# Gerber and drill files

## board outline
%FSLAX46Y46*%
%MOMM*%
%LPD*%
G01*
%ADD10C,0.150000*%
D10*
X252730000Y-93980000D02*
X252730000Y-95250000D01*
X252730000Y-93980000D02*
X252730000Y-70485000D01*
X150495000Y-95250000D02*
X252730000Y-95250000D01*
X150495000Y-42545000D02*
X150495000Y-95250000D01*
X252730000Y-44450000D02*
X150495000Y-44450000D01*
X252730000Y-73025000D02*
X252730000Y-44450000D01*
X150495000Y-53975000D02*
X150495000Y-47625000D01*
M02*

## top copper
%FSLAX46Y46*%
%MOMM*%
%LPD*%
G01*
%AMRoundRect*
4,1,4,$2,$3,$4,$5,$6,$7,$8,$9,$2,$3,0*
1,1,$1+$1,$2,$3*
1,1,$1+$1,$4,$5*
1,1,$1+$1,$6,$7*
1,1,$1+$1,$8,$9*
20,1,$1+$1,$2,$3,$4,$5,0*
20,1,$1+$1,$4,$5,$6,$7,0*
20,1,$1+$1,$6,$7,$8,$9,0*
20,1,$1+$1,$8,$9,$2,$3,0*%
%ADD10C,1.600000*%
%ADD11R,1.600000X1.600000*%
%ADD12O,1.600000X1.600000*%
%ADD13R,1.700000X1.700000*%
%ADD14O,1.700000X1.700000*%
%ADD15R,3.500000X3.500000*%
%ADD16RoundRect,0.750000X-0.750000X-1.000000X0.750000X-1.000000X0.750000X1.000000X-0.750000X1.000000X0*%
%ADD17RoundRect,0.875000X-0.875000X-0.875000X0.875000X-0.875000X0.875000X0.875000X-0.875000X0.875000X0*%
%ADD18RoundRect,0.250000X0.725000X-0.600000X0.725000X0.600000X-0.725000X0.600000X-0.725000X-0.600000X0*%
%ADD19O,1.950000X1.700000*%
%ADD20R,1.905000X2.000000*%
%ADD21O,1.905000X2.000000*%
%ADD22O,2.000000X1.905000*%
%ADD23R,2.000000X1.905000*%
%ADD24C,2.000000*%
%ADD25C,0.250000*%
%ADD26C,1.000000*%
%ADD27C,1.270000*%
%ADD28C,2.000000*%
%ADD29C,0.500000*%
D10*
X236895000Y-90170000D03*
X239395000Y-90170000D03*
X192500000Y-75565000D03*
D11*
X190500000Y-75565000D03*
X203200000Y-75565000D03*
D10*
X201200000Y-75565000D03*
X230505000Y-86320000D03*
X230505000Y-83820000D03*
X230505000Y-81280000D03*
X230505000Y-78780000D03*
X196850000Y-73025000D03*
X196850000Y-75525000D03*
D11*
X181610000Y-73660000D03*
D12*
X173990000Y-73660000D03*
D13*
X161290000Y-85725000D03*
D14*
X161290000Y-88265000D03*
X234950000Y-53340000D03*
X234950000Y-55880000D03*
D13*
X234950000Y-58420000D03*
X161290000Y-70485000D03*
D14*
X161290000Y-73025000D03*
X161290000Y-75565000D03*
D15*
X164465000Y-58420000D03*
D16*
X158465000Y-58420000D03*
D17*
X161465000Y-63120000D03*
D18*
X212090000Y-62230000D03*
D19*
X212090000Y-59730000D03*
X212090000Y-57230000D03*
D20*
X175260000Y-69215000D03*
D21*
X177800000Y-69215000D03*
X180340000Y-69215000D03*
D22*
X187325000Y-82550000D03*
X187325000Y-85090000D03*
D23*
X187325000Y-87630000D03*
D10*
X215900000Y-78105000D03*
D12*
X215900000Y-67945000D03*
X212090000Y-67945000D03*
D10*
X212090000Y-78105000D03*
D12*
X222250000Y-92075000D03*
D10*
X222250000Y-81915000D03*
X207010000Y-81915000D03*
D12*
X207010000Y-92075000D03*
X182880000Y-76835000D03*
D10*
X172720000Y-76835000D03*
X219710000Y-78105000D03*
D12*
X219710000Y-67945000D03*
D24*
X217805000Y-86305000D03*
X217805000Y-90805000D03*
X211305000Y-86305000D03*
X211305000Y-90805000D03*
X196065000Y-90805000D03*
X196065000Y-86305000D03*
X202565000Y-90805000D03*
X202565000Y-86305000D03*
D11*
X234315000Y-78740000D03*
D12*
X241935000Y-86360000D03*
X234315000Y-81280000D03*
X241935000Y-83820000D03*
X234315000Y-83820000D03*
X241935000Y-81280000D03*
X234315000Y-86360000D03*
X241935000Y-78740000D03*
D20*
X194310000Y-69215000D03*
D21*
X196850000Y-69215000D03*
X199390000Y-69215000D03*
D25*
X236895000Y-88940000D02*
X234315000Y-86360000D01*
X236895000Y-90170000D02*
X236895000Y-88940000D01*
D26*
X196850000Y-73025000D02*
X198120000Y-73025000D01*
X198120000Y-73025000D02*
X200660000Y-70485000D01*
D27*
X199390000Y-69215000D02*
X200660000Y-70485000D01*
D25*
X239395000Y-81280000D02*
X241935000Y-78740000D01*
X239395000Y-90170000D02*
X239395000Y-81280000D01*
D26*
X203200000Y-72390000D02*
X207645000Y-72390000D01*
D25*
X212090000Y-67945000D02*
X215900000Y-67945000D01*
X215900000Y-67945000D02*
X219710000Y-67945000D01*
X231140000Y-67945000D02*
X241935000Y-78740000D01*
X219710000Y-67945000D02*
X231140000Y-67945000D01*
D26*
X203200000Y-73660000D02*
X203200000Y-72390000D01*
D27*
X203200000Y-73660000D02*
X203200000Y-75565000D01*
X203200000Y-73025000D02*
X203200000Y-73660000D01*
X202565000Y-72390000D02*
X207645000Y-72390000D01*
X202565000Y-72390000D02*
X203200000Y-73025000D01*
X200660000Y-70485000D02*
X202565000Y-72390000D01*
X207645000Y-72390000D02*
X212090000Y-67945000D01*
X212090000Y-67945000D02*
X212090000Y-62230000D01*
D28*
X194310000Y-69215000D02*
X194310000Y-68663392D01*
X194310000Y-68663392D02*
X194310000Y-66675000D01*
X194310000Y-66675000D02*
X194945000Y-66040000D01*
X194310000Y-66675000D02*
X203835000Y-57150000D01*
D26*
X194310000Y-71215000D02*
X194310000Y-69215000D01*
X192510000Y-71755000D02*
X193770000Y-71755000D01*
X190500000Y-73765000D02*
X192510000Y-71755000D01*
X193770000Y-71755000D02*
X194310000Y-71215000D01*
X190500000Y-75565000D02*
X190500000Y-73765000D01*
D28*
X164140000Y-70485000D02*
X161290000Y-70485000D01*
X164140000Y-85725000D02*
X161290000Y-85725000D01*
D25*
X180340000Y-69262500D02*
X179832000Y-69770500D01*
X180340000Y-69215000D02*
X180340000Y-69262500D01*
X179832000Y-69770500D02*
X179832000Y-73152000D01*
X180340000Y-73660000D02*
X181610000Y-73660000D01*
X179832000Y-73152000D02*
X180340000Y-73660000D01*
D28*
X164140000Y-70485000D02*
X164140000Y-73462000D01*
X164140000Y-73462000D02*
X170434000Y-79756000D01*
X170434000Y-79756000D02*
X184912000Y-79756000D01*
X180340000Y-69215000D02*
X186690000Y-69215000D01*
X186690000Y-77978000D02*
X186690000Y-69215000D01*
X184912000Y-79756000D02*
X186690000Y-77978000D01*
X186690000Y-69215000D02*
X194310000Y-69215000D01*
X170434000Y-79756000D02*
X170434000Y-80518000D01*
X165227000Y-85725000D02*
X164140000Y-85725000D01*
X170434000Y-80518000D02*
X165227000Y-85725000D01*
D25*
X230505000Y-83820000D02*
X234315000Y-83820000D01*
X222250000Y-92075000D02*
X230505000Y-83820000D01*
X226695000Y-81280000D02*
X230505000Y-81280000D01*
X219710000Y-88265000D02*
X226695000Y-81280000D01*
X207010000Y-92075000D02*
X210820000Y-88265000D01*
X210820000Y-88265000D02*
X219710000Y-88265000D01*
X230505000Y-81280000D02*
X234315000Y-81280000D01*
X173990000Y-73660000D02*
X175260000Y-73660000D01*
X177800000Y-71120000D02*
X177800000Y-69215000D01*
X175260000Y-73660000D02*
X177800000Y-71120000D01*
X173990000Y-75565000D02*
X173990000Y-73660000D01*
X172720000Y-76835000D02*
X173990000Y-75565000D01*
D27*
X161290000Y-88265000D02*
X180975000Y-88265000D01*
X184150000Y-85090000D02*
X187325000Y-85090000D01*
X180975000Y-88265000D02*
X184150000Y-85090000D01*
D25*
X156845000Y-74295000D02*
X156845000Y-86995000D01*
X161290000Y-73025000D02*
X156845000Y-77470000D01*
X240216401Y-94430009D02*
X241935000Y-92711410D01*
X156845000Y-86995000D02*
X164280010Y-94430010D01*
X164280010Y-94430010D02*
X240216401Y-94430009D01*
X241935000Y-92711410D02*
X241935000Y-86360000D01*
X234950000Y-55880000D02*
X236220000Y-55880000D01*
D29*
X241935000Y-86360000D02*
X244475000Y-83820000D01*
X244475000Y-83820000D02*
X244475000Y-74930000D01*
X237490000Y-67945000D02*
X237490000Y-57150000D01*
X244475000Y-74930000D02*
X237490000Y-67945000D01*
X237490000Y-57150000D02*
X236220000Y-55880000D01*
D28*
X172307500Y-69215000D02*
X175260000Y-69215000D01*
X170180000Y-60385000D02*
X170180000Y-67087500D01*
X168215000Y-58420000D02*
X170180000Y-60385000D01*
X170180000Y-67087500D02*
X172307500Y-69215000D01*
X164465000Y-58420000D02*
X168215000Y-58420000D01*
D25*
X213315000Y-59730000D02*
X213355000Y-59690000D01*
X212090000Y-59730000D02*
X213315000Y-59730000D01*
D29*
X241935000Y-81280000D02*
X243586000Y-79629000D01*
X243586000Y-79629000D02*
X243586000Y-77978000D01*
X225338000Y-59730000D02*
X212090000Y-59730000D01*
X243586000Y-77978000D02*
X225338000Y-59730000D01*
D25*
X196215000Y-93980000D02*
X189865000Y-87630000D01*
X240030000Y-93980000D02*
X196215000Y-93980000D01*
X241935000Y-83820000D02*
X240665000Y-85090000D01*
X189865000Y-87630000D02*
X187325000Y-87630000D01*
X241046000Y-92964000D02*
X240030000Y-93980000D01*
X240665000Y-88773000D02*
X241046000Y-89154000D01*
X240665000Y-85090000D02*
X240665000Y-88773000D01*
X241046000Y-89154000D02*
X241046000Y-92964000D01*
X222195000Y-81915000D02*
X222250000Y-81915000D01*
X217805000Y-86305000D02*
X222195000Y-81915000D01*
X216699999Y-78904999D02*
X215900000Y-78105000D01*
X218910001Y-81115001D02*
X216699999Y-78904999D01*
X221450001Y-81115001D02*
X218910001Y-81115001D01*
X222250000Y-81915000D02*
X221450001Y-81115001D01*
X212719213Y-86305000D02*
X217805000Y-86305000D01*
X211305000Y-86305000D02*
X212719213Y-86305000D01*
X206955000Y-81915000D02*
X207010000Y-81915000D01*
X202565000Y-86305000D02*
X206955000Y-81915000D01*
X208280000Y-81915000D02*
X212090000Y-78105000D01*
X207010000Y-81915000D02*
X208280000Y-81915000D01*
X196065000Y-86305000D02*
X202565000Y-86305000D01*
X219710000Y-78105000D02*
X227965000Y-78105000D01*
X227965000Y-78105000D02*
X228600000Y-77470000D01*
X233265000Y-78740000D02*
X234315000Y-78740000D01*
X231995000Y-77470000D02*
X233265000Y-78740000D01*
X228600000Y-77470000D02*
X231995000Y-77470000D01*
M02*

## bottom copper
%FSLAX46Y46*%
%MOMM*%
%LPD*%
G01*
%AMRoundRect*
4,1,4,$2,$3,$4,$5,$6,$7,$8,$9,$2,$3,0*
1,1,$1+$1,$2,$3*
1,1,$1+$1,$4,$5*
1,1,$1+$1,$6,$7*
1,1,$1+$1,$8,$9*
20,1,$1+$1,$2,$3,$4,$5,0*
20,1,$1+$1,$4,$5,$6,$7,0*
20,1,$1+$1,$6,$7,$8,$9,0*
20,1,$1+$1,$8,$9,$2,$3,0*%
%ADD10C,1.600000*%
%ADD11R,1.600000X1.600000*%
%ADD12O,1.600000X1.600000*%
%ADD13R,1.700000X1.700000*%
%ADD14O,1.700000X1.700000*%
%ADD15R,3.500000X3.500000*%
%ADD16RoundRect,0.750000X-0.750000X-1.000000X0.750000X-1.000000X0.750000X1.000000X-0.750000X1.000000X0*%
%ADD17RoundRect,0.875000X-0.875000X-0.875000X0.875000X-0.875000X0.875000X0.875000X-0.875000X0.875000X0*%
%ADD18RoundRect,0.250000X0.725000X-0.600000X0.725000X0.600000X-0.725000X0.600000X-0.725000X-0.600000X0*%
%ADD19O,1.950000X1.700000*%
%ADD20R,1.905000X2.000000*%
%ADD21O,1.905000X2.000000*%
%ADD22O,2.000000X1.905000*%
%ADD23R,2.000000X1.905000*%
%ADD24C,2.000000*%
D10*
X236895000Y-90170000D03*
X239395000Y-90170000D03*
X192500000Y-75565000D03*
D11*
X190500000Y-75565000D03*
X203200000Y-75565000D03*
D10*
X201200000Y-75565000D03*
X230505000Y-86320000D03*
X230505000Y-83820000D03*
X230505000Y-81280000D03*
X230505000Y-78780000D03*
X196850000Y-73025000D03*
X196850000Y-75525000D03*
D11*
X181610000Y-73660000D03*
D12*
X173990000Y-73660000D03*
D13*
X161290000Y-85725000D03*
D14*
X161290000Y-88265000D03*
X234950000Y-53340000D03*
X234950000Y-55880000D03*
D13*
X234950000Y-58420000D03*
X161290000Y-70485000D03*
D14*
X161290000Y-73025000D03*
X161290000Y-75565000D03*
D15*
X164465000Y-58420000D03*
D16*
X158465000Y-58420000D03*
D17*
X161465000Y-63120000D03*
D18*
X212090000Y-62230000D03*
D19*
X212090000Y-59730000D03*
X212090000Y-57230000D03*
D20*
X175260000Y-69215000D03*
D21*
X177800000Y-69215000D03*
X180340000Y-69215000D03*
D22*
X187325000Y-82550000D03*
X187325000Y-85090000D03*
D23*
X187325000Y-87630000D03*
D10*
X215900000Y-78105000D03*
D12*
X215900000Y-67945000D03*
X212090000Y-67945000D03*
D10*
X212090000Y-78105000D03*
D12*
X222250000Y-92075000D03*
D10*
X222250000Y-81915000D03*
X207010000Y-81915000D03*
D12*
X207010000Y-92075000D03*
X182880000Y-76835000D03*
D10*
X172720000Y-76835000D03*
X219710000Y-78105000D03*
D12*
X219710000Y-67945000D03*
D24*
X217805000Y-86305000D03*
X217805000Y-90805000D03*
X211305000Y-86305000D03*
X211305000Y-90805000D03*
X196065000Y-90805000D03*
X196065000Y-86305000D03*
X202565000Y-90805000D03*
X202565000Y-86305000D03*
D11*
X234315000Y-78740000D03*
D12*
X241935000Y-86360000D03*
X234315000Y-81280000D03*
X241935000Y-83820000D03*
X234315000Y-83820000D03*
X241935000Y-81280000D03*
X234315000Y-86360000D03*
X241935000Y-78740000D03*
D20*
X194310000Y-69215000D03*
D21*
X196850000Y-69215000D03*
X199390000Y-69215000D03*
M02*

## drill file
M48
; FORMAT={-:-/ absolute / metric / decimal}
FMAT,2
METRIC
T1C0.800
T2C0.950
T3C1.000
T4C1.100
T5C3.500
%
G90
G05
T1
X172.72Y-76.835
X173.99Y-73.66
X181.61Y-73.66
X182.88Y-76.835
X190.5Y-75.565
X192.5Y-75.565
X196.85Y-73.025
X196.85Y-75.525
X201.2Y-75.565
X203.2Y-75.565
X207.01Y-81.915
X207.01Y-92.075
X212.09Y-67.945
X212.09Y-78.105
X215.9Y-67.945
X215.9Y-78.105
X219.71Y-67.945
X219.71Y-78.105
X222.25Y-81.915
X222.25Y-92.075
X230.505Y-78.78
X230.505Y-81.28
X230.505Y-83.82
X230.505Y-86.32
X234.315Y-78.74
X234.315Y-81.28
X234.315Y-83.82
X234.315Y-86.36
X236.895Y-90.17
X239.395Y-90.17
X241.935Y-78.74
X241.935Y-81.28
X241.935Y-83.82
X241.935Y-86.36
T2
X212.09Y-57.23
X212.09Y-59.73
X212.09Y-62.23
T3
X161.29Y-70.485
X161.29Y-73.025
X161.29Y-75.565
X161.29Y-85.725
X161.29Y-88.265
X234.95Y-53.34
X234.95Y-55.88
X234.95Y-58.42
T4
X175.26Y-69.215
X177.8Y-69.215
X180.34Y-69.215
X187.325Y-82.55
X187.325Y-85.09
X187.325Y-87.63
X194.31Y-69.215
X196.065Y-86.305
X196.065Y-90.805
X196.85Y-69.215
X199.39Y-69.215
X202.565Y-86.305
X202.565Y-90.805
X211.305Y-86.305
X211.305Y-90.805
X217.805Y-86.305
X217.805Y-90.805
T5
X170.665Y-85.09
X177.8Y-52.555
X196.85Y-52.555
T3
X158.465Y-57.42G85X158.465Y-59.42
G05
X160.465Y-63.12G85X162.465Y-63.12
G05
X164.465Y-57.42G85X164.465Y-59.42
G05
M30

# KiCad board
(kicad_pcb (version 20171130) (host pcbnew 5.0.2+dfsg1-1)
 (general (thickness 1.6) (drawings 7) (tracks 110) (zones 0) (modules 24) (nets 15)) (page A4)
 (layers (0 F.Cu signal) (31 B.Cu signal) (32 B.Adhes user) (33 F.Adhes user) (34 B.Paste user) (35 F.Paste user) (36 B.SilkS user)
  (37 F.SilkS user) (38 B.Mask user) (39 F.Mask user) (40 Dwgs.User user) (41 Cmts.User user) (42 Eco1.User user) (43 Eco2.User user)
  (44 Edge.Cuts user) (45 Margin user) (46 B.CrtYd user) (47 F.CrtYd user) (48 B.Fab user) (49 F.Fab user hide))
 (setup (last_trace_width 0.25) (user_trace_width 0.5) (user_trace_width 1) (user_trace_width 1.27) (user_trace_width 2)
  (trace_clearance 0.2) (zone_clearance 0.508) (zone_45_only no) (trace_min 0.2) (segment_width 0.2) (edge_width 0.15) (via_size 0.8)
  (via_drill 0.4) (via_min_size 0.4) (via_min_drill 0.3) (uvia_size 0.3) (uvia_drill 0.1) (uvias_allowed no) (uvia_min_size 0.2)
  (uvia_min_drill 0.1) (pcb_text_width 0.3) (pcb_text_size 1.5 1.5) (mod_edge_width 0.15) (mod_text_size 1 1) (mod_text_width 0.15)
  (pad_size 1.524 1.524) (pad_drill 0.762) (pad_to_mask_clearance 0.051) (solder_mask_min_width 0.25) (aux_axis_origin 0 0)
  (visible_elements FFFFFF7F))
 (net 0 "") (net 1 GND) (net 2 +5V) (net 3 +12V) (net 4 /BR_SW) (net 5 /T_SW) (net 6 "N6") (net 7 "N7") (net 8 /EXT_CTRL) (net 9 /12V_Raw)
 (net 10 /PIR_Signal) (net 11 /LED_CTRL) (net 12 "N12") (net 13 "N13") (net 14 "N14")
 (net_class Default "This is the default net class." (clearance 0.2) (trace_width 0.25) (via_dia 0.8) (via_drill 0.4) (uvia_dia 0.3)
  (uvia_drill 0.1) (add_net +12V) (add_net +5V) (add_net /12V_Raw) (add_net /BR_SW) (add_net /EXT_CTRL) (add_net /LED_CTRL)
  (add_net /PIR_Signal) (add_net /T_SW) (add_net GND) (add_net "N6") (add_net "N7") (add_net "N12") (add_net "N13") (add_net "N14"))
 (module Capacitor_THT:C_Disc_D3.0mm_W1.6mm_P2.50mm (layer F.Cu) (at 239.395 90.17 180)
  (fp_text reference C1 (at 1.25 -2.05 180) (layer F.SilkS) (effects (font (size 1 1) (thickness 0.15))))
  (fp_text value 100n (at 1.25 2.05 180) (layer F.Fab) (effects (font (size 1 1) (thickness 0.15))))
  (pad 2 thru_hole circle (at 2.5 0 180) (size 1.6 1.6) (drill 0.8) (layers *.Cu *.Mask) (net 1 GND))
  (pad 1 thru_hole circle (at 0 0 180) (size 1.6 1.6) (drill 0.8) (layers *.Cu *.Mask) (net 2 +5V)))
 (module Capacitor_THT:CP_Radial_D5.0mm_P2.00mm (layer F.Cu) (at 190.5 75.565)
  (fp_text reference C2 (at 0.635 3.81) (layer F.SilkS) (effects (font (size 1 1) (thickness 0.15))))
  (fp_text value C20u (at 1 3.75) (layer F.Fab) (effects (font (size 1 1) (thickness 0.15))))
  (pad 2 thru_hole circle (at 2 0) (size 1.6 1.6) (drill 0.8) (layers *.Cu *.Mask) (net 1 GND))
  (pad 1 thru_hole rect (at 0 0) (size 1.6 1.6) (drill 0.8) (layers *.Cu *.Mask) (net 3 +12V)))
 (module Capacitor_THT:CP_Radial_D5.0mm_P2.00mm (layer F.Cu) (at 203.2 75.565 180)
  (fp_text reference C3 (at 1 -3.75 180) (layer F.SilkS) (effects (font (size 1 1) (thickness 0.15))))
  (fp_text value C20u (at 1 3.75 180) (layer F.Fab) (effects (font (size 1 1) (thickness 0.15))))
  (pad 1 thru_hole rect (at 0 0 180) (size 1.6 1.6) (drill 0.8) (layers *.Cu *.Mask) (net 2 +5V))
  (pad 2 thru_hole circle (at 2 0 180) (size 1.6 1.6) (drill 0.8) (layers *.Cu *.Mask) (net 1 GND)))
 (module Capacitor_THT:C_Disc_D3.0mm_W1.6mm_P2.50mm (layer F.Cu) (at 230.505 83.82 270)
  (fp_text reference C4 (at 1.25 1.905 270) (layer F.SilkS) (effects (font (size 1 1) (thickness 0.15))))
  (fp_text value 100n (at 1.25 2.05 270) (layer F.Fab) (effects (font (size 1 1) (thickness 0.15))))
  (pad 2 thru_hole circle (at 2.5 0 270) (size 1.6 1.6) (drill 0.8) (layers *.Cu *.Mask) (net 1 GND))
  (pad 1 thru_hole circle (at 0 0 270) (size 1.6 1.6) (drill 0.8) (layers *.Cu *.Mask) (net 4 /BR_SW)))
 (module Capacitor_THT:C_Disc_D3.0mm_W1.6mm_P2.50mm (layer F.Cu) (at 230.505 81.28 90)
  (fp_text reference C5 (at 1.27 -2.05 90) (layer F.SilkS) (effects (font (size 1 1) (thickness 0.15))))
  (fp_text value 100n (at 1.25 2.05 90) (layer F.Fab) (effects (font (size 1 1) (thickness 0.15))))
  (pad 1 thru_hole circle (at 0 0 90) (size 1.6 1.6) (drill 0.8) (layers *.Cu *.Mask) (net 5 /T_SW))
  (pad 2 thru_hole circle (at 2.5 0 90) (size 1.6 1.6) (drill 0.8) (layers *.Cu *.Mask) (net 1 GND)))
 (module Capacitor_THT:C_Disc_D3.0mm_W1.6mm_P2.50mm (layer F.Cu) (at 196.85 73.025 270)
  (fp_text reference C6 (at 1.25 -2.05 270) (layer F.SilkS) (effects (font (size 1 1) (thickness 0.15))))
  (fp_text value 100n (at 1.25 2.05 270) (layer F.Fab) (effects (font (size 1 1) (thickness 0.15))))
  (pad 1 thru_hole circle (at 0 0 270) (size 1.6 1.6) (drill 0.8) (layers *.Cu *.Mask) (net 2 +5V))
  (pad 2 thru_hole circle (at 2.5 0 270) (size 1.6 1.6) (drill 0.8) (layers *.Cu *.Mask) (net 1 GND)))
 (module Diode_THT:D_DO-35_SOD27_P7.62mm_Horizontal (layer F.Cu) (at 181.61 73.66 180)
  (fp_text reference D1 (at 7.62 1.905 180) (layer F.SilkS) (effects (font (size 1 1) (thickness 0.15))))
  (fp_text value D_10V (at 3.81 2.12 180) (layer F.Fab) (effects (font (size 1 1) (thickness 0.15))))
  (pad 1 thru_hole rect (at 0 0 180) (size 1.6 1.6) (drill 0.8) (layers *.Cu *.Mask) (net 3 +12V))
  (pad 2 thru_hole oval (at 7.62 0 180) (size 1.6 1.6) (drill 0.8) (layers *.Cu *.Mask) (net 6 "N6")))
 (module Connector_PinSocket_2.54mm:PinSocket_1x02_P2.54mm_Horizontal (layer F.Cu) (at 161.29 85.725)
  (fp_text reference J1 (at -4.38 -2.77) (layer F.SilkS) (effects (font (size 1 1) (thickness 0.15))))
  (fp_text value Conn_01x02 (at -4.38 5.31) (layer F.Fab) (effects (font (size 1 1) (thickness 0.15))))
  (pad 1 thru_hole rect (at 0 0) (size 1.7 1.7) (drill 1) (layers *.Cu *.Mask) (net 3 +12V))
  (pad 2 thru_hole oval (at 0 2.54) (size 1.7 1.7) (drill 1) (layers *.Cu *.Mask) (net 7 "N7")))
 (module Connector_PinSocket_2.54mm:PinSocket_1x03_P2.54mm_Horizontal (layer F.Cu) (at 234.95 58.42 180)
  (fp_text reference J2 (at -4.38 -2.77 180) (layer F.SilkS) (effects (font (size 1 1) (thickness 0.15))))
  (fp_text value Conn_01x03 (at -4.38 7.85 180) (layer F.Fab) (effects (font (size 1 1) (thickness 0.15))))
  (pad 3 thru_hole oval (at 0 5.08 180) (size 1.7 1.7) (drill 1) (layers *.Cu *.Mask) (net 1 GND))
  (pad 2 thru_hole oval (at 0 2.54 180) (size 1.7 1.7) (drill 1) (layers *.Cu *.Mask) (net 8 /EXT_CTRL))
  (pad 1 thru_hole rect (at 0 0 180) (size 1.7 1.7) (drill 1) (layers *.Cu *.Mask) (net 3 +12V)))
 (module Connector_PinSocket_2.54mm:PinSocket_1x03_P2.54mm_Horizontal (layer F.Cu) (at 161.29 70.485)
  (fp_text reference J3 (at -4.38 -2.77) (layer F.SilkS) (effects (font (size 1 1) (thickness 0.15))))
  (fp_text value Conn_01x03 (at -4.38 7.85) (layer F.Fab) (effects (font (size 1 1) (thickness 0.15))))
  (pad 1 thru_hole rect (at 0 0) (size 1.7 1.7) (drill 1) (layers *.Cu *.Mask) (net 3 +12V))
  (pad 2 thru_hole oval (at 0 2.54) (size 1.7 1.7) (drill 1) (layers *.Cu *.Mask) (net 8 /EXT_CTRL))
  (pad 3 thru_hole oval (at 0 5.08) (size 1.7 1.7) (drill 1) (layers *.Cu *.Mask) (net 1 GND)))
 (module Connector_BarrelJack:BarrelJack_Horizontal (layer F.Cu) (at 164.465 58.42)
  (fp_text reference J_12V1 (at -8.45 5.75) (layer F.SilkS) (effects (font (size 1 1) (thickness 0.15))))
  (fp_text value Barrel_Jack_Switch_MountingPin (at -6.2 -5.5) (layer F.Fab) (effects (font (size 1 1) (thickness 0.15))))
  (pad 1 thru_hole rect (at 0 0) (size 3.5 3.5) (drill oval 1 3) (layers *.Cu *.Mask) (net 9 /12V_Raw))
  (pad 2 thru_hole roundrect (at -6 0) (size 3 3.5) (drill oval 1 3) (layers *.Cu *.Mask) (roundrect_rratio 0.25) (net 1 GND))
  (pad 3 thru_hole roundrect (at -3 4.7) (size 3.5 3.5) (drill oval 3 1) (layers *.Cu *.Mask) (roundrect_rratio 0.25) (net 1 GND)))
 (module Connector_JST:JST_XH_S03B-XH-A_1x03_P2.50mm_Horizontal (layer F.Cu) (at 212.09 62.23 90)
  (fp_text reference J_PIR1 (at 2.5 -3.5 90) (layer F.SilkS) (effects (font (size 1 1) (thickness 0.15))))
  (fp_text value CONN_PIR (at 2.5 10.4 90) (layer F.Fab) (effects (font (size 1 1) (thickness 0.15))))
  (pad 1 thru_hole roundrect (at 0 0 90) (size 1.7 1.95) (drill 0.95) (layers *.Cu *.Mask) (roundrect_rratio 0.147059) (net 2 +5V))
  (pad 2 thru_hole oval (at 2.5 0 90) (size 1.7 1.95) (drill 0.95) (layers *.Cu *.Mask) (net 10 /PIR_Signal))
  (pad 3 thru_hole oval (at 5 0 90) (size 1.7 1.95) (drill 0.95) (layers *.Cu *.Mask) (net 1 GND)))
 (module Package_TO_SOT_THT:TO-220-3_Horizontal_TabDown (layer F.Cu) (at 175.26 69.215)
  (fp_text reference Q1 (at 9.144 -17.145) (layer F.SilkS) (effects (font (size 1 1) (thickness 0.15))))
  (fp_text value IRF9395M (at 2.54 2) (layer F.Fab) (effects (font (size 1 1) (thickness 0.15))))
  (pad "" np_thru_hole oval (at 2.54 -16.66) (size 3.5 3.5) (drill 3.5) (layers *.Cu *.Mask))
  (pad 1 thru_hole rect (at 0 0) (size 1.905 2) (drill 1.1) (layers *.Cu *.Mask) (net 9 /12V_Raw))
  (pad 2 thru_hole oval (at 2.54 0) (size 1.905 2) (drill 1.1) (layers *.Cu *.Mask) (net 6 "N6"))
  (pad 3 thru_hole oval (at 5.08 0) (size 1.905 2) (drill 1.1) (layers *.Cu *.Mask) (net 3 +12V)))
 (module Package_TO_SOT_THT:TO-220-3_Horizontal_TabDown (layer F.Cu) (at 187.325 87.63 90)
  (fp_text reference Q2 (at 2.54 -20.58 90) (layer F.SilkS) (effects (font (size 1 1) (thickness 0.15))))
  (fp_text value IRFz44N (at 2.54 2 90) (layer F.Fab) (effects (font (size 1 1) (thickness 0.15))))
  (pad 3 thru_hole oval (at 5.08 0 90) (size 1.905 2) (drill 1.1) (layers *.Cu *.Mask) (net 1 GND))
  (pad 2 thru_hole oval (at 2.54 0 90) (size 1.905 2) (drill 1.1) (layers *.Cu *.Mask) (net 7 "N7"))
  (pad 1 thru_hole rect (at 0 0 90) (size 1.905 2) (drill 1.1) (layers *.Cu *.Mask) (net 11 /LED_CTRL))
  (pad "" np_thru_hole oval (at 2.54 -16.66 90) (size 3.5 3.5) (drill 3.5) (layers *.Cu *.Mask)))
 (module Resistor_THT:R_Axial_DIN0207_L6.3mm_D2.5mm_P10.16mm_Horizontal (layer F.Cu) (at 215.9 78.105 90)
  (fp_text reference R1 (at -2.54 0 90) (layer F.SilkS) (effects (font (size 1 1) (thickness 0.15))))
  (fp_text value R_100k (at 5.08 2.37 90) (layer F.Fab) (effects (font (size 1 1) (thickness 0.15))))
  (pad 1 thru_hole circle (at 0 0 90) (size 1.6 1.6) (drill 0.8) (layers *.Cu *.Mask) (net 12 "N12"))
  (pad 2 thru_hole oval (at 10.16 0 90) (size 1.6 1.6) (drill 0.8) (layers *.Cu *.Mask) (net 2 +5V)))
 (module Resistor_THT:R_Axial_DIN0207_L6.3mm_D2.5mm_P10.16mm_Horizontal (layer F.Cu) (at 212.09 78.105 90)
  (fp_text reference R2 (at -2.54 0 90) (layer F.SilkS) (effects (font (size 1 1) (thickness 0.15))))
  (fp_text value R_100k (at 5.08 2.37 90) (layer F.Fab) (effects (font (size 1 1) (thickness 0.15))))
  (pad 2 thru_hole oval (at 10.16 0 90) (size 1.6 1.6) (drill 0.8) (layers *.Cu *.Mask) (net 2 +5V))
  (pad 1 thru_hole circle (at 0 0 90) (size 1.6 1.6) (drill 0.8) (layers *.Cu *.Mask) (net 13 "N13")))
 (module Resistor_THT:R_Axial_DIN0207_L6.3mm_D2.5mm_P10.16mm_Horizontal (layer F.Cu) (at 222.25 81.915 270)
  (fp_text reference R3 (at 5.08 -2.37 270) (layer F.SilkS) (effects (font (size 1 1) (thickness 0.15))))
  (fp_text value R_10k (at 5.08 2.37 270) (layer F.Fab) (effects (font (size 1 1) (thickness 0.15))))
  (pad 2 thru_hole oval (at 10.16 0 270) (size 1.6 1.6) (drill 0.8) (layers *.Cu *.Mask) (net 4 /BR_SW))
  (pad 1 thru_hole circle (at 0 0 270) (size 1.6 1.6) (drill 0.8) (layers *.Cu *.Mask) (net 12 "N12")))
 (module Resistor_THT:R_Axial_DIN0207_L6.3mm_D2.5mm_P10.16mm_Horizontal (layer F.Cu) (at 207.01 81.915 270)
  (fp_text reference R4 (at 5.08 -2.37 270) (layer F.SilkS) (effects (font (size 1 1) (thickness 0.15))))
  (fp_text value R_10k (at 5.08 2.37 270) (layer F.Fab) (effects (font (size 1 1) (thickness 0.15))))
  (pad 1 thru_hole circle (at 0 0 270) (size 1.6 1.6) (drill 0.8) (layers *.Cu *.Mask) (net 13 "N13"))
  (pad 2 thru_hole oval (at 10.16 0 270) (size 1.6 1.6) (drill 0.8) (layers *.Cu *.Mask) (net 5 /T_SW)))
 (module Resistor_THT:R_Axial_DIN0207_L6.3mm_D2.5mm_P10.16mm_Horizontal (layer F.Cu) (at 172.72 76.835)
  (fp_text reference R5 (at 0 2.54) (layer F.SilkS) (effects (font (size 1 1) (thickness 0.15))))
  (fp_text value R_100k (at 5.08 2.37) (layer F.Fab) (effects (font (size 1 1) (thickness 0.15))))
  (pad 2 thru_hole oval (at 10.16 0) (size 1.6 1.6) (drill 0.8) (layers *.Cu *.Mask) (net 1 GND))
  (pad 1 thru_hole circle (at 0 0) (size 1.6 1.6) (drill 0.8) (layers *.Cu *.Mask) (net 6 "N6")))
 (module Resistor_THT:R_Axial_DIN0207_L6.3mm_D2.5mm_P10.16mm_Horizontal (layer F.Cu) (at 219.71 78.105 90)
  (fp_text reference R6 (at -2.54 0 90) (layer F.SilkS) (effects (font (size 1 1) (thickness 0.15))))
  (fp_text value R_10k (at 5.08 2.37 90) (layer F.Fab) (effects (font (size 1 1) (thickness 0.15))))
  (pad 1 thru_hole circle (at 0 0 90) (size 1.6 1.6) (drill 0.8) (layers *.Cu *.Mask) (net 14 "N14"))
  (pad 2 thru_hole oval (at 10.16 0 90) (size 1.6 1.6) (drill 0.8) (layers *.Cu *.Mask) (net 2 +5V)))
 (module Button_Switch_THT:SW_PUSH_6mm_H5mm (layer F.Cu) (at 217.805 90.805 180)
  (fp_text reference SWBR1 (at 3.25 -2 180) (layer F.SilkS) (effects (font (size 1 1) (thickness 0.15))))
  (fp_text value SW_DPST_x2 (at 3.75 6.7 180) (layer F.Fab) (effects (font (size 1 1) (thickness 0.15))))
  (pad 2 thru_hole circle (at 0 4.5 270) (size 2 2) (drill 1.1) (layers *.Cu *.Mask) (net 12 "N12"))
  (pad 1 thru_hole circle (at 0 0 270) (size 2 2) (drill 1.1) (layers *.Cu *.Mask) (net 1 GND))
  (pad 2 thru_hole circle (at 6.5 4.5 270) (size 2 2) (drill 1.1) (layers *.Cu *.Mask) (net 12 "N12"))
  (pad 1 thru_hole circle (at 6.5 0 270) (size 2 2) (drill 1.1) (layers *.Cu *.Mask) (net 1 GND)))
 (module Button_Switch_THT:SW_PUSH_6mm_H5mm (layer F.Cu) (at 202.565 90.805 180)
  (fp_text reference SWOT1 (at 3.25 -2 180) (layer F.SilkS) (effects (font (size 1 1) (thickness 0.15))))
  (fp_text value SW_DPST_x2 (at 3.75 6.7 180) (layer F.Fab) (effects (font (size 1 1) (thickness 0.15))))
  (pad 1 thru_hole circle (at 6.5 0 270) (size 2 2) (drill 1.1) (layers *.Cu *.Mask) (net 1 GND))
  (pad 2 thru_hole circle (at 6.5 4.5 270) (size 2 2) (drill 1.1) (layers *.Cu *.Mask) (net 13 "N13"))
  (pad 1 thru_hole circle (at 0 0 270) (size 2 2) (drill 1.1) (layers *.Cu *.Mask) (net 1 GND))
  (pad 2 thru_hole circle (at 0 4.5 270) (size 2 2) (drill 1.1) (layers *.Cu *.Mask) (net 13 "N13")))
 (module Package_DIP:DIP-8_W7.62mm (layer F.Cu) (at 234.315 78.74)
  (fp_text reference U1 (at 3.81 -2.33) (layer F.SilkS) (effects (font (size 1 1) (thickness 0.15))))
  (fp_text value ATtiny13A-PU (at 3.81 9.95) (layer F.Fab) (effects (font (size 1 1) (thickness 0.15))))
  (pad 1 thru_hole rect (at 0 0) (size 1.6 1.6) (drill 0.8) (layers *.Cu *.Mask) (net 14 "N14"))
  (pad 5 thru_hole oval (at 7.62 7.62) (size 1.6 1.6) (drill 0.8) (layers *.Cu *.Mask) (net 8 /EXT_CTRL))
  (pad 2 thru_hole oval (at 0 2.54) (size 1.6 1.6) (drill 0.8) (layers *.Cu *.Mask) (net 5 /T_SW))
  (pad 6 thru_hole oval (at 7.62 5.08) (size 1.6 1.6) (drill 0.8) (layers *.Cu *.Mask) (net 11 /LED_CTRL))
  (pad 3 thru_hole oval (at 0 5.08) (size 1.6 1.6) (drill 0.8) (layers *.Cu *.Mask) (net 4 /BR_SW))
  (pad 7 thru_hole oval (at 7.62 2.54) (size 1.6 1.6) (drill 0.8) (layers *.Cu *.Mask) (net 10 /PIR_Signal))
  (pad 4 thru_hole oval (at 0 7.62) (size 1.6 1.6) (drill 0.8) (layers *.Cu *.Mask) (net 1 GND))
  (pad 8 thru_hole oval (at 7.62 0) (size 1.6 1.6) (drill 0.8) (layers *.Cu *.Mask) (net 2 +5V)))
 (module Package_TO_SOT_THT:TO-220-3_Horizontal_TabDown (layer F.Cu) (at 194.31 69.215)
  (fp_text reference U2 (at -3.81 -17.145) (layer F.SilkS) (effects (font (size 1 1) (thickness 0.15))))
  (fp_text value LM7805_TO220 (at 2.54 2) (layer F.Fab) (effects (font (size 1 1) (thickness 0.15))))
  (pad "" np_thru_hole oval (at 2.54 -16.66) (size 3.5 3.5) (drill 3.5) (layers *.Cu *.Mask))
  (pad 1 thru_hole rect (at 0 0) (size 1.905 2) (drill 1.1) (layers *.Cu *.Mask) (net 3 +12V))
  (pad 2 thru_hole oval (at 2.54 0) (size 1.905 2) (drill 1.1) (layers *.Cu *.Mask) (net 1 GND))
  (pad 3 thru_hole oval (at 5.08 0) (size 1.905 2) (drill 1.1) (layers *.Cu *.Mask) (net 2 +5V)))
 (gr_line (start 252.73 93.98) (end 252.73 95.25) (layer Edge.Cuts) (width 0.15))
 (gr_line (start 252.73 93.98) (end 252.73 70.485) (layer Edge.Cuts) (width 0.15))
 (gr_line (start 150.495 95.25) (end 252.73 95.25) (layer Edge.Cuts) (width 0.15))
 (gr_line (start 150.495 42.545) (end 150.495 95.25) (layer Edge.Cuts) (width 0.15))
 (gr_line (start 252.73 44.45) (end 150.495 44.45) (layer Edge.Cuts) (width 0.15))
 (gr_line (start 252.73 73.025) (end 252.73 44.45) (layer Edge.Cuts) (width 0.15))
 (gr_line (start 150.495 53.975) (end 150.495 47.625) (layer Edge.Cuts) (width 0.15))
 (segment (start 236.895 88.94) (end 234.315 86.36) (width 0.25) (layer F.Cu) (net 1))
 (segment (start 236.895 90.17) (end 236.895 88.94) (width 0.25) (layer F.Cu) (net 1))
 (segment (start 196.85 73.025) (end 198.12 73.025) (width 1) (layer F.Cu) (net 2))
 (segment (start 198.12 73.025) (end 200.66 70.485) (width 1) (layer F.Cu) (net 2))
 (segment (start 199.39 69.215) (end 200.66 70.485) (width 1.27) (layer F.Cu) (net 2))
 (segment (start 239.395 81.28) (end 241.935 78.74) (width 0.25) (layer F.Cu) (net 2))
 (segment (start 239.395 90.17) (end 239.395 81.28) (width 0.25) (layer F.Cu) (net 2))
 (segment (start 203.2 72.39) (end 207.645 72.39) (width 1) (layer F.Cu) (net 2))
 (segment (start 212.09 67.945) (end 215.9 67.945) (width 0.25) (layer F.Cu) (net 2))
 (segment (start 215.9 67.945) (end 219.71 67.945) (width 0.25) (layer F.Cu) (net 2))
 (segment (start 231.14 67.945) (end 241.935 78.74) (width 0.25) (layer F.Cu) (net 2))
 (segment (start 219.71 67.945) (end 231.14 67.945) (width 0.25) (layer F.Cu) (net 2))
 (segment (start 203.2 73.66) (end 203.2 72.39) (width 1) (layer F.Cu) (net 2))
 (segment (start 203.2 73.66) (end 203.2 75.565) (width 1.27) (layer F.Cu) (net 2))
 (segment (start 203.2 73.025) (end 203.2 73.66) (width 1.27) (layer F.Cu) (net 2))
 (segment (start 202.565 72.39) (end 207.645 72.39) (width 1.27) (layer F.Cu) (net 2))
 (segment (start 202.565 72.39) (end 203.2 73.025) (width 1.27) (layer F.Cu) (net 2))
 (segment (start 200.66 70.485) (end 202.565 72.39) (width 1.27) (layer F.Cu) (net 2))
 (segment (start 207.645 72.39) (end 212.09 67.945) (width 1.27) (layer F.Cu) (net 2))
 (segment (start 212.09 67.945) (end 212.09 62.23) (width 1.27) (layer F.Cu) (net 2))
 (segment (start 194.31 69.215) (end 194.31 68.663392) (width 2) (layer F.Cu) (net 3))
 (segment (start 194.31 68.663392) (end 194.31 66.675) (width 2) (layer F.Cu) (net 3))
 (segment (start 194.31 66.675) (end 194.945 66.04) (width 2) (layer F.Cu) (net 3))
 (segment (start 194.31 66.675) (end 203.835 57.15) (width 2) (layer F.Cu) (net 3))
 (segment (start 194.31 71.215) (end 194.31 69.215) (width 1) (layer F.Cu) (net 3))
 (segment (start 192.51 71.755) (end 193.77 71.755) (width 1) (layer F.Cu) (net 3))
 (segment (start 190.5 73.765) (end 192.51 71.755) (width 1) (layer F.Cu) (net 3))
 (segment (start 193.77 71.755) (end 194.31 71.215) (width 1) (layer F.Cu) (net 3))
 (segment (start 190.5 75.565) (end 190.5 73.765) (width 1) (layer F.Cu) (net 3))
 (segment (start 164.14 70.485) (end 161.29 70.485) (width 2) (layer F.Cu) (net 3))
 (segment (start 164.14 85.725) (end 161.29 85.725) (width 2) (layer F.Cu) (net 3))
 (segment (start 180.34 69.2625) (end 179.832 69.7705) (width 0.25) (layer F.Cu) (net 3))
 (segment (start 180.34 69.215) (end 180.34 69.2625) (width 0.25) (layer F.Cu) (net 3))
 (segment (start 179.832 69.7705) (end 179.832 73.152) (width 0.25) (layer F.Cu) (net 3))
 (segment (start 180.34 73.66) (end 181.61 73.66) (width 0.25) (layer F.Cu) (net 3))
 (segment (start 179.832 73.152) (end 180.34 73.66) (width 0.25) (layer F.Cu) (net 3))
 (segment (start 164.14 70.485) (end 164.14 73.462) (width 2) (layer F.Cu) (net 3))
 (segment (start 164.14 73.462) (end 170.434 79.756) (width 2) (layer F.Cu) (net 3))
 (segment (start 170.434 79.756) (end 184.912 79.756) (width 2) (layer F.Cu) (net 3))
 (segment (start 180.34 69.215) (end 186.69 69.215) (width 2) (layer F.Cu) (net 3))
 (segment (start 186.69 77.978) (end 186.69 69.215) (width 2) (layer F.Cu) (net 3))
 (segment (start 184.912 79.756) (end 186.69 77.978) (width 2) (layer F.Cu) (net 3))
 (segment (start 186.69 69.215) (end 194.31 69.215) (width 2) (layer F.Cu) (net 3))
 (segment (start 170.434 79.756) (end 170.434 80.518) (width 2) (layer F.Cu) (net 3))
 (segment (start 165.227 85.725) (end 164.14 85.725) (width 2) (layer F.Cu) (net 3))
 (segment (start 170.434 80.518) (end 165.227 85.725) (width 2) (layer F.Cu) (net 3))
 (segment (start 230.505 83.82) (end 234.315 83.82) (width 0.25) (layer F.Cu) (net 4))
 (segment (start 222.25 92.075) (end 230.505 83.82) (width 0.25) (layer F.Cu) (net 4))
 (segment (start 226.695 81.28) (end 230.505 81.28) (width 0.25) (layer F.Cu) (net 5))
 (segment (start 219.71 88.265) (end 226.695 81.28) (width 0.25) (layer F.Cu) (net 5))
 (segment (start 207.01 92.075) (end 210.82 88.265) (width 0.25) (layer F.Cu) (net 5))
 (segment (start 210.82 88.265) (end 219.71 88.265) (width 0.25) (layer F.Cu) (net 5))
 (segment (start 230.505 81.28) (end 234.315 81.28) (width 0.25) (layer F.Cu) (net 5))
 (segment (start 173.99 73.66) (end 175.26 73.66) (width 0.25) (layer F.Cu) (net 6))
 (segment (start 177.8 71.12) (end 177.8 69.215) (width 0.25) (layer F.Cu) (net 6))
 (segment (start 175.26 73.66) (end 177.8 71.12) (width 0.25) (layer F.Cu) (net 6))
 (segment (start 173.99 75.565) (end 173.99 73.66) (width 0.25) (layer F.Cu) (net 6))
 (segment (start 172.72 76.835) (end 173.99 75.565) (width 0.25) (layer F.Cu) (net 6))
 (segment (start 161.29 88.265) (end 180.975 88.265) (width 1.27) (layer F.Cu) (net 7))
 (segment (start 184.15 85.09) (end 187.325 85.09) (width 1.27) (layer F.Cu) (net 7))
 (segment (start 180.975 88.265) (end 184.15 85.09) (width 1.27) (layer F.Cu) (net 7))
 (segment (start 156.845 74.295) (end 156.845 86.995) (width 0.25) (layer F.Cu) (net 8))
 (segment (start 161.29 73.025) (end 156.845 77.47) (width 0.25) (layer F.Cu) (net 8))
 (segment (start 240.216401 94.430009) (end 241.935 92.71141) (width 0.25) (layer F.Cu) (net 8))
 (segment (start 156.845 86.995) (end 164.28001 94.43001) (width 0.25) (layer F.Cu) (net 8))
 (segment (start 164.28001 94.43001) (end 240.216401 94.430009) (width 0.25) (layer F.Cu) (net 8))
 (segment (start 241.935 92.71141) (end 241.935 86.36) (width 0.25) (layer F.Cu) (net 8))
 (segment (start 234.95 55.88) (end 236.22 55.88) (width 0.25) (layer F.Cu) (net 8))
 (segment (start 241.935 86.36) (end 244.475 83.82) (width 0.5) (layer F.Cu) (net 8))
 (segment (start 244.475 83.82) (end 244.475 74.93) (width 0.5) (layer F.Cu) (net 8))
 (segment (start 237.49 67.945) (end 237.49 57.15) (width 0.5) (layer F.Cu) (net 8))
 (segment (start 244.475 74.93) (end 237.49 67.945) (width 0.5) (layer F.Cu) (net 8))
 (segment (start 237.49 57.15) (end 236.22 55.88) (width 0.5) (layer F.Cu) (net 8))
 (segment (start 172.3075 69.215) (end 175.26 69.215) (width 2) (layer F.Cu) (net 9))
 (segment (start 170.18 60.385) (end 170.18 67.0875) (width 2) (layer F.Cu) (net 9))
 (segment (start 168.215 58.42) (end 170.18 60.385) (width 2) (layer F.Cu) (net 9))
 (segment (start 170.18 67.0875) (end 172.3075 69.215) (width 2) (layer F.Cu) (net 9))
 (segment (start 164.465 58.42) (end 168.215 58.42) (width 2) (layer F.Cu) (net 9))
 (segment (start 213.315 59.73) (end 213.355 59.69) (width 0.25) (layer F.Cu) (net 10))
 (segment (start 212.09 59.73) (end 213.315 59.73) (width 0.25) (layer F.Cu) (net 10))
 (segment (start 241.935 81.28) (end 243.586 79.629) (width 0.5) (layer F.Cu) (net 10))
 (segment (start 243.586 79.629) (end 243.586 77.978) (width 0.5) (layer F.Cu) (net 10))
 (segment (start 225.338 59.73) (end 212.09 59.73) (width 0.5) (layer F.Cu) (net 10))
 (segment (start 243.586 77.978) (end 225.338 59.73) (width 0.5) (layer F.Cu) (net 10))
 (segment (start 196.215 93.98) (end 189.865 87.63) (width 0.25) (layer F.Cu) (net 11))
 (segment (start 240.03 93.98) (end 196.215 93.98) (width 0.25) (layer F.Cu) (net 11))
 (segment (start 241.935 83.82) (end 240.665 85.09) (width 0.25) (layer F.Cu) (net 11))
 (segment (start 189.865 87.63) (end 187.325 87.63) (width 0.25) (layer F.Cu) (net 11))
 (segment (start 241.046 92.964) (end 240.03 93.98) (width 0.25) (layer F.Cu) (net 11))
 (segment (start 240.665 88.773) (end 241.046 89.154) (width 0.25) (layer F.Cu) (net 11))
 (segment (start 240.665 85.09) (end 240.665 88.773) (width 0.25) (layer F.Cu) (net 11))
 (segment (start 241.046 89.154) (end 241.046 92.964) (width 0.25) (layer F.Cu) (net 11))
 (segment (start 222.195 81.915) (end 222.25 81.915) (width 0.25) (layer F.Cu) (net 12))
 (segment (start 217.805 86.305) (end 222.195 81.915) (width 0.25) (layer F.Cu) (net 12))
 (segment (start 216.699999 78.904999) (end 215.9 78.105) (width 0.25) (layer F.Cu) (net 12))
 (segment (start 218.910001 81.115001) (end 216.699999 78.904999) (width 0.25) (layer F.Cu) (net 12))
 (segment (start 221.450001 81.115001) (end 218.910001 81.115001) (width 0.25) (layer F.Cu) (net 12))
 (segment (start 222.25 81.915) (end 221.450001 81.115001) (width 0.25) (layer F.Cu) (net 12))
 (segment (start 212.719213 86.305) (end 217.805 86.305) (width 0.25) (layer F.Cu) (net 12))
 (segment (start 211.305 86.305) (end 212.719213 86.305) (width 0.25) (layer F.Cu) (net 12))
 (segment (start 206.955 81.915) (end 207.01 81.915) (width 0.25) (layer F.Cu) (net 13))
 (segment (start 202.565 86.305) (end 206.955 81.915) (width 0.25) (layer F.Cu) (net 13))
 (segment (start 208.28 81.915) (end 212.09 78.105) (width 0.25) (layer F.Cu) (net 13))
 (segment (start 207.01 81.915) (end 208.28 81.915) (width 0.25) (layer F.Cu) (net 13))
 (segment (start 196.065 86.305) (end 202.565 86.305) (width 0.25) (layer F.Cu) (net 13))
 (segment (start 219.71 78.105) (end 227.965 78.105) (width 0.25) (layer F.Cu) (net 14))
 (segment (start 227.965 78.105) (end 228.6 77.47) (width 0.25) (layer F.Cu) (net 14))
 (segment (start 233.265 78.74) (end 234.315 78.74) (width 0.25) (layer F.Cu) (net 14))
 (segment (start 231.995 77.47) (end 233.265 78.74) (width 0.25) (layer F.Cu) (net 14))
 (segment (start 228.6 77.47) (end 231.995 77.47) (width 0.25) (layer F.Cu) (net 14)))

